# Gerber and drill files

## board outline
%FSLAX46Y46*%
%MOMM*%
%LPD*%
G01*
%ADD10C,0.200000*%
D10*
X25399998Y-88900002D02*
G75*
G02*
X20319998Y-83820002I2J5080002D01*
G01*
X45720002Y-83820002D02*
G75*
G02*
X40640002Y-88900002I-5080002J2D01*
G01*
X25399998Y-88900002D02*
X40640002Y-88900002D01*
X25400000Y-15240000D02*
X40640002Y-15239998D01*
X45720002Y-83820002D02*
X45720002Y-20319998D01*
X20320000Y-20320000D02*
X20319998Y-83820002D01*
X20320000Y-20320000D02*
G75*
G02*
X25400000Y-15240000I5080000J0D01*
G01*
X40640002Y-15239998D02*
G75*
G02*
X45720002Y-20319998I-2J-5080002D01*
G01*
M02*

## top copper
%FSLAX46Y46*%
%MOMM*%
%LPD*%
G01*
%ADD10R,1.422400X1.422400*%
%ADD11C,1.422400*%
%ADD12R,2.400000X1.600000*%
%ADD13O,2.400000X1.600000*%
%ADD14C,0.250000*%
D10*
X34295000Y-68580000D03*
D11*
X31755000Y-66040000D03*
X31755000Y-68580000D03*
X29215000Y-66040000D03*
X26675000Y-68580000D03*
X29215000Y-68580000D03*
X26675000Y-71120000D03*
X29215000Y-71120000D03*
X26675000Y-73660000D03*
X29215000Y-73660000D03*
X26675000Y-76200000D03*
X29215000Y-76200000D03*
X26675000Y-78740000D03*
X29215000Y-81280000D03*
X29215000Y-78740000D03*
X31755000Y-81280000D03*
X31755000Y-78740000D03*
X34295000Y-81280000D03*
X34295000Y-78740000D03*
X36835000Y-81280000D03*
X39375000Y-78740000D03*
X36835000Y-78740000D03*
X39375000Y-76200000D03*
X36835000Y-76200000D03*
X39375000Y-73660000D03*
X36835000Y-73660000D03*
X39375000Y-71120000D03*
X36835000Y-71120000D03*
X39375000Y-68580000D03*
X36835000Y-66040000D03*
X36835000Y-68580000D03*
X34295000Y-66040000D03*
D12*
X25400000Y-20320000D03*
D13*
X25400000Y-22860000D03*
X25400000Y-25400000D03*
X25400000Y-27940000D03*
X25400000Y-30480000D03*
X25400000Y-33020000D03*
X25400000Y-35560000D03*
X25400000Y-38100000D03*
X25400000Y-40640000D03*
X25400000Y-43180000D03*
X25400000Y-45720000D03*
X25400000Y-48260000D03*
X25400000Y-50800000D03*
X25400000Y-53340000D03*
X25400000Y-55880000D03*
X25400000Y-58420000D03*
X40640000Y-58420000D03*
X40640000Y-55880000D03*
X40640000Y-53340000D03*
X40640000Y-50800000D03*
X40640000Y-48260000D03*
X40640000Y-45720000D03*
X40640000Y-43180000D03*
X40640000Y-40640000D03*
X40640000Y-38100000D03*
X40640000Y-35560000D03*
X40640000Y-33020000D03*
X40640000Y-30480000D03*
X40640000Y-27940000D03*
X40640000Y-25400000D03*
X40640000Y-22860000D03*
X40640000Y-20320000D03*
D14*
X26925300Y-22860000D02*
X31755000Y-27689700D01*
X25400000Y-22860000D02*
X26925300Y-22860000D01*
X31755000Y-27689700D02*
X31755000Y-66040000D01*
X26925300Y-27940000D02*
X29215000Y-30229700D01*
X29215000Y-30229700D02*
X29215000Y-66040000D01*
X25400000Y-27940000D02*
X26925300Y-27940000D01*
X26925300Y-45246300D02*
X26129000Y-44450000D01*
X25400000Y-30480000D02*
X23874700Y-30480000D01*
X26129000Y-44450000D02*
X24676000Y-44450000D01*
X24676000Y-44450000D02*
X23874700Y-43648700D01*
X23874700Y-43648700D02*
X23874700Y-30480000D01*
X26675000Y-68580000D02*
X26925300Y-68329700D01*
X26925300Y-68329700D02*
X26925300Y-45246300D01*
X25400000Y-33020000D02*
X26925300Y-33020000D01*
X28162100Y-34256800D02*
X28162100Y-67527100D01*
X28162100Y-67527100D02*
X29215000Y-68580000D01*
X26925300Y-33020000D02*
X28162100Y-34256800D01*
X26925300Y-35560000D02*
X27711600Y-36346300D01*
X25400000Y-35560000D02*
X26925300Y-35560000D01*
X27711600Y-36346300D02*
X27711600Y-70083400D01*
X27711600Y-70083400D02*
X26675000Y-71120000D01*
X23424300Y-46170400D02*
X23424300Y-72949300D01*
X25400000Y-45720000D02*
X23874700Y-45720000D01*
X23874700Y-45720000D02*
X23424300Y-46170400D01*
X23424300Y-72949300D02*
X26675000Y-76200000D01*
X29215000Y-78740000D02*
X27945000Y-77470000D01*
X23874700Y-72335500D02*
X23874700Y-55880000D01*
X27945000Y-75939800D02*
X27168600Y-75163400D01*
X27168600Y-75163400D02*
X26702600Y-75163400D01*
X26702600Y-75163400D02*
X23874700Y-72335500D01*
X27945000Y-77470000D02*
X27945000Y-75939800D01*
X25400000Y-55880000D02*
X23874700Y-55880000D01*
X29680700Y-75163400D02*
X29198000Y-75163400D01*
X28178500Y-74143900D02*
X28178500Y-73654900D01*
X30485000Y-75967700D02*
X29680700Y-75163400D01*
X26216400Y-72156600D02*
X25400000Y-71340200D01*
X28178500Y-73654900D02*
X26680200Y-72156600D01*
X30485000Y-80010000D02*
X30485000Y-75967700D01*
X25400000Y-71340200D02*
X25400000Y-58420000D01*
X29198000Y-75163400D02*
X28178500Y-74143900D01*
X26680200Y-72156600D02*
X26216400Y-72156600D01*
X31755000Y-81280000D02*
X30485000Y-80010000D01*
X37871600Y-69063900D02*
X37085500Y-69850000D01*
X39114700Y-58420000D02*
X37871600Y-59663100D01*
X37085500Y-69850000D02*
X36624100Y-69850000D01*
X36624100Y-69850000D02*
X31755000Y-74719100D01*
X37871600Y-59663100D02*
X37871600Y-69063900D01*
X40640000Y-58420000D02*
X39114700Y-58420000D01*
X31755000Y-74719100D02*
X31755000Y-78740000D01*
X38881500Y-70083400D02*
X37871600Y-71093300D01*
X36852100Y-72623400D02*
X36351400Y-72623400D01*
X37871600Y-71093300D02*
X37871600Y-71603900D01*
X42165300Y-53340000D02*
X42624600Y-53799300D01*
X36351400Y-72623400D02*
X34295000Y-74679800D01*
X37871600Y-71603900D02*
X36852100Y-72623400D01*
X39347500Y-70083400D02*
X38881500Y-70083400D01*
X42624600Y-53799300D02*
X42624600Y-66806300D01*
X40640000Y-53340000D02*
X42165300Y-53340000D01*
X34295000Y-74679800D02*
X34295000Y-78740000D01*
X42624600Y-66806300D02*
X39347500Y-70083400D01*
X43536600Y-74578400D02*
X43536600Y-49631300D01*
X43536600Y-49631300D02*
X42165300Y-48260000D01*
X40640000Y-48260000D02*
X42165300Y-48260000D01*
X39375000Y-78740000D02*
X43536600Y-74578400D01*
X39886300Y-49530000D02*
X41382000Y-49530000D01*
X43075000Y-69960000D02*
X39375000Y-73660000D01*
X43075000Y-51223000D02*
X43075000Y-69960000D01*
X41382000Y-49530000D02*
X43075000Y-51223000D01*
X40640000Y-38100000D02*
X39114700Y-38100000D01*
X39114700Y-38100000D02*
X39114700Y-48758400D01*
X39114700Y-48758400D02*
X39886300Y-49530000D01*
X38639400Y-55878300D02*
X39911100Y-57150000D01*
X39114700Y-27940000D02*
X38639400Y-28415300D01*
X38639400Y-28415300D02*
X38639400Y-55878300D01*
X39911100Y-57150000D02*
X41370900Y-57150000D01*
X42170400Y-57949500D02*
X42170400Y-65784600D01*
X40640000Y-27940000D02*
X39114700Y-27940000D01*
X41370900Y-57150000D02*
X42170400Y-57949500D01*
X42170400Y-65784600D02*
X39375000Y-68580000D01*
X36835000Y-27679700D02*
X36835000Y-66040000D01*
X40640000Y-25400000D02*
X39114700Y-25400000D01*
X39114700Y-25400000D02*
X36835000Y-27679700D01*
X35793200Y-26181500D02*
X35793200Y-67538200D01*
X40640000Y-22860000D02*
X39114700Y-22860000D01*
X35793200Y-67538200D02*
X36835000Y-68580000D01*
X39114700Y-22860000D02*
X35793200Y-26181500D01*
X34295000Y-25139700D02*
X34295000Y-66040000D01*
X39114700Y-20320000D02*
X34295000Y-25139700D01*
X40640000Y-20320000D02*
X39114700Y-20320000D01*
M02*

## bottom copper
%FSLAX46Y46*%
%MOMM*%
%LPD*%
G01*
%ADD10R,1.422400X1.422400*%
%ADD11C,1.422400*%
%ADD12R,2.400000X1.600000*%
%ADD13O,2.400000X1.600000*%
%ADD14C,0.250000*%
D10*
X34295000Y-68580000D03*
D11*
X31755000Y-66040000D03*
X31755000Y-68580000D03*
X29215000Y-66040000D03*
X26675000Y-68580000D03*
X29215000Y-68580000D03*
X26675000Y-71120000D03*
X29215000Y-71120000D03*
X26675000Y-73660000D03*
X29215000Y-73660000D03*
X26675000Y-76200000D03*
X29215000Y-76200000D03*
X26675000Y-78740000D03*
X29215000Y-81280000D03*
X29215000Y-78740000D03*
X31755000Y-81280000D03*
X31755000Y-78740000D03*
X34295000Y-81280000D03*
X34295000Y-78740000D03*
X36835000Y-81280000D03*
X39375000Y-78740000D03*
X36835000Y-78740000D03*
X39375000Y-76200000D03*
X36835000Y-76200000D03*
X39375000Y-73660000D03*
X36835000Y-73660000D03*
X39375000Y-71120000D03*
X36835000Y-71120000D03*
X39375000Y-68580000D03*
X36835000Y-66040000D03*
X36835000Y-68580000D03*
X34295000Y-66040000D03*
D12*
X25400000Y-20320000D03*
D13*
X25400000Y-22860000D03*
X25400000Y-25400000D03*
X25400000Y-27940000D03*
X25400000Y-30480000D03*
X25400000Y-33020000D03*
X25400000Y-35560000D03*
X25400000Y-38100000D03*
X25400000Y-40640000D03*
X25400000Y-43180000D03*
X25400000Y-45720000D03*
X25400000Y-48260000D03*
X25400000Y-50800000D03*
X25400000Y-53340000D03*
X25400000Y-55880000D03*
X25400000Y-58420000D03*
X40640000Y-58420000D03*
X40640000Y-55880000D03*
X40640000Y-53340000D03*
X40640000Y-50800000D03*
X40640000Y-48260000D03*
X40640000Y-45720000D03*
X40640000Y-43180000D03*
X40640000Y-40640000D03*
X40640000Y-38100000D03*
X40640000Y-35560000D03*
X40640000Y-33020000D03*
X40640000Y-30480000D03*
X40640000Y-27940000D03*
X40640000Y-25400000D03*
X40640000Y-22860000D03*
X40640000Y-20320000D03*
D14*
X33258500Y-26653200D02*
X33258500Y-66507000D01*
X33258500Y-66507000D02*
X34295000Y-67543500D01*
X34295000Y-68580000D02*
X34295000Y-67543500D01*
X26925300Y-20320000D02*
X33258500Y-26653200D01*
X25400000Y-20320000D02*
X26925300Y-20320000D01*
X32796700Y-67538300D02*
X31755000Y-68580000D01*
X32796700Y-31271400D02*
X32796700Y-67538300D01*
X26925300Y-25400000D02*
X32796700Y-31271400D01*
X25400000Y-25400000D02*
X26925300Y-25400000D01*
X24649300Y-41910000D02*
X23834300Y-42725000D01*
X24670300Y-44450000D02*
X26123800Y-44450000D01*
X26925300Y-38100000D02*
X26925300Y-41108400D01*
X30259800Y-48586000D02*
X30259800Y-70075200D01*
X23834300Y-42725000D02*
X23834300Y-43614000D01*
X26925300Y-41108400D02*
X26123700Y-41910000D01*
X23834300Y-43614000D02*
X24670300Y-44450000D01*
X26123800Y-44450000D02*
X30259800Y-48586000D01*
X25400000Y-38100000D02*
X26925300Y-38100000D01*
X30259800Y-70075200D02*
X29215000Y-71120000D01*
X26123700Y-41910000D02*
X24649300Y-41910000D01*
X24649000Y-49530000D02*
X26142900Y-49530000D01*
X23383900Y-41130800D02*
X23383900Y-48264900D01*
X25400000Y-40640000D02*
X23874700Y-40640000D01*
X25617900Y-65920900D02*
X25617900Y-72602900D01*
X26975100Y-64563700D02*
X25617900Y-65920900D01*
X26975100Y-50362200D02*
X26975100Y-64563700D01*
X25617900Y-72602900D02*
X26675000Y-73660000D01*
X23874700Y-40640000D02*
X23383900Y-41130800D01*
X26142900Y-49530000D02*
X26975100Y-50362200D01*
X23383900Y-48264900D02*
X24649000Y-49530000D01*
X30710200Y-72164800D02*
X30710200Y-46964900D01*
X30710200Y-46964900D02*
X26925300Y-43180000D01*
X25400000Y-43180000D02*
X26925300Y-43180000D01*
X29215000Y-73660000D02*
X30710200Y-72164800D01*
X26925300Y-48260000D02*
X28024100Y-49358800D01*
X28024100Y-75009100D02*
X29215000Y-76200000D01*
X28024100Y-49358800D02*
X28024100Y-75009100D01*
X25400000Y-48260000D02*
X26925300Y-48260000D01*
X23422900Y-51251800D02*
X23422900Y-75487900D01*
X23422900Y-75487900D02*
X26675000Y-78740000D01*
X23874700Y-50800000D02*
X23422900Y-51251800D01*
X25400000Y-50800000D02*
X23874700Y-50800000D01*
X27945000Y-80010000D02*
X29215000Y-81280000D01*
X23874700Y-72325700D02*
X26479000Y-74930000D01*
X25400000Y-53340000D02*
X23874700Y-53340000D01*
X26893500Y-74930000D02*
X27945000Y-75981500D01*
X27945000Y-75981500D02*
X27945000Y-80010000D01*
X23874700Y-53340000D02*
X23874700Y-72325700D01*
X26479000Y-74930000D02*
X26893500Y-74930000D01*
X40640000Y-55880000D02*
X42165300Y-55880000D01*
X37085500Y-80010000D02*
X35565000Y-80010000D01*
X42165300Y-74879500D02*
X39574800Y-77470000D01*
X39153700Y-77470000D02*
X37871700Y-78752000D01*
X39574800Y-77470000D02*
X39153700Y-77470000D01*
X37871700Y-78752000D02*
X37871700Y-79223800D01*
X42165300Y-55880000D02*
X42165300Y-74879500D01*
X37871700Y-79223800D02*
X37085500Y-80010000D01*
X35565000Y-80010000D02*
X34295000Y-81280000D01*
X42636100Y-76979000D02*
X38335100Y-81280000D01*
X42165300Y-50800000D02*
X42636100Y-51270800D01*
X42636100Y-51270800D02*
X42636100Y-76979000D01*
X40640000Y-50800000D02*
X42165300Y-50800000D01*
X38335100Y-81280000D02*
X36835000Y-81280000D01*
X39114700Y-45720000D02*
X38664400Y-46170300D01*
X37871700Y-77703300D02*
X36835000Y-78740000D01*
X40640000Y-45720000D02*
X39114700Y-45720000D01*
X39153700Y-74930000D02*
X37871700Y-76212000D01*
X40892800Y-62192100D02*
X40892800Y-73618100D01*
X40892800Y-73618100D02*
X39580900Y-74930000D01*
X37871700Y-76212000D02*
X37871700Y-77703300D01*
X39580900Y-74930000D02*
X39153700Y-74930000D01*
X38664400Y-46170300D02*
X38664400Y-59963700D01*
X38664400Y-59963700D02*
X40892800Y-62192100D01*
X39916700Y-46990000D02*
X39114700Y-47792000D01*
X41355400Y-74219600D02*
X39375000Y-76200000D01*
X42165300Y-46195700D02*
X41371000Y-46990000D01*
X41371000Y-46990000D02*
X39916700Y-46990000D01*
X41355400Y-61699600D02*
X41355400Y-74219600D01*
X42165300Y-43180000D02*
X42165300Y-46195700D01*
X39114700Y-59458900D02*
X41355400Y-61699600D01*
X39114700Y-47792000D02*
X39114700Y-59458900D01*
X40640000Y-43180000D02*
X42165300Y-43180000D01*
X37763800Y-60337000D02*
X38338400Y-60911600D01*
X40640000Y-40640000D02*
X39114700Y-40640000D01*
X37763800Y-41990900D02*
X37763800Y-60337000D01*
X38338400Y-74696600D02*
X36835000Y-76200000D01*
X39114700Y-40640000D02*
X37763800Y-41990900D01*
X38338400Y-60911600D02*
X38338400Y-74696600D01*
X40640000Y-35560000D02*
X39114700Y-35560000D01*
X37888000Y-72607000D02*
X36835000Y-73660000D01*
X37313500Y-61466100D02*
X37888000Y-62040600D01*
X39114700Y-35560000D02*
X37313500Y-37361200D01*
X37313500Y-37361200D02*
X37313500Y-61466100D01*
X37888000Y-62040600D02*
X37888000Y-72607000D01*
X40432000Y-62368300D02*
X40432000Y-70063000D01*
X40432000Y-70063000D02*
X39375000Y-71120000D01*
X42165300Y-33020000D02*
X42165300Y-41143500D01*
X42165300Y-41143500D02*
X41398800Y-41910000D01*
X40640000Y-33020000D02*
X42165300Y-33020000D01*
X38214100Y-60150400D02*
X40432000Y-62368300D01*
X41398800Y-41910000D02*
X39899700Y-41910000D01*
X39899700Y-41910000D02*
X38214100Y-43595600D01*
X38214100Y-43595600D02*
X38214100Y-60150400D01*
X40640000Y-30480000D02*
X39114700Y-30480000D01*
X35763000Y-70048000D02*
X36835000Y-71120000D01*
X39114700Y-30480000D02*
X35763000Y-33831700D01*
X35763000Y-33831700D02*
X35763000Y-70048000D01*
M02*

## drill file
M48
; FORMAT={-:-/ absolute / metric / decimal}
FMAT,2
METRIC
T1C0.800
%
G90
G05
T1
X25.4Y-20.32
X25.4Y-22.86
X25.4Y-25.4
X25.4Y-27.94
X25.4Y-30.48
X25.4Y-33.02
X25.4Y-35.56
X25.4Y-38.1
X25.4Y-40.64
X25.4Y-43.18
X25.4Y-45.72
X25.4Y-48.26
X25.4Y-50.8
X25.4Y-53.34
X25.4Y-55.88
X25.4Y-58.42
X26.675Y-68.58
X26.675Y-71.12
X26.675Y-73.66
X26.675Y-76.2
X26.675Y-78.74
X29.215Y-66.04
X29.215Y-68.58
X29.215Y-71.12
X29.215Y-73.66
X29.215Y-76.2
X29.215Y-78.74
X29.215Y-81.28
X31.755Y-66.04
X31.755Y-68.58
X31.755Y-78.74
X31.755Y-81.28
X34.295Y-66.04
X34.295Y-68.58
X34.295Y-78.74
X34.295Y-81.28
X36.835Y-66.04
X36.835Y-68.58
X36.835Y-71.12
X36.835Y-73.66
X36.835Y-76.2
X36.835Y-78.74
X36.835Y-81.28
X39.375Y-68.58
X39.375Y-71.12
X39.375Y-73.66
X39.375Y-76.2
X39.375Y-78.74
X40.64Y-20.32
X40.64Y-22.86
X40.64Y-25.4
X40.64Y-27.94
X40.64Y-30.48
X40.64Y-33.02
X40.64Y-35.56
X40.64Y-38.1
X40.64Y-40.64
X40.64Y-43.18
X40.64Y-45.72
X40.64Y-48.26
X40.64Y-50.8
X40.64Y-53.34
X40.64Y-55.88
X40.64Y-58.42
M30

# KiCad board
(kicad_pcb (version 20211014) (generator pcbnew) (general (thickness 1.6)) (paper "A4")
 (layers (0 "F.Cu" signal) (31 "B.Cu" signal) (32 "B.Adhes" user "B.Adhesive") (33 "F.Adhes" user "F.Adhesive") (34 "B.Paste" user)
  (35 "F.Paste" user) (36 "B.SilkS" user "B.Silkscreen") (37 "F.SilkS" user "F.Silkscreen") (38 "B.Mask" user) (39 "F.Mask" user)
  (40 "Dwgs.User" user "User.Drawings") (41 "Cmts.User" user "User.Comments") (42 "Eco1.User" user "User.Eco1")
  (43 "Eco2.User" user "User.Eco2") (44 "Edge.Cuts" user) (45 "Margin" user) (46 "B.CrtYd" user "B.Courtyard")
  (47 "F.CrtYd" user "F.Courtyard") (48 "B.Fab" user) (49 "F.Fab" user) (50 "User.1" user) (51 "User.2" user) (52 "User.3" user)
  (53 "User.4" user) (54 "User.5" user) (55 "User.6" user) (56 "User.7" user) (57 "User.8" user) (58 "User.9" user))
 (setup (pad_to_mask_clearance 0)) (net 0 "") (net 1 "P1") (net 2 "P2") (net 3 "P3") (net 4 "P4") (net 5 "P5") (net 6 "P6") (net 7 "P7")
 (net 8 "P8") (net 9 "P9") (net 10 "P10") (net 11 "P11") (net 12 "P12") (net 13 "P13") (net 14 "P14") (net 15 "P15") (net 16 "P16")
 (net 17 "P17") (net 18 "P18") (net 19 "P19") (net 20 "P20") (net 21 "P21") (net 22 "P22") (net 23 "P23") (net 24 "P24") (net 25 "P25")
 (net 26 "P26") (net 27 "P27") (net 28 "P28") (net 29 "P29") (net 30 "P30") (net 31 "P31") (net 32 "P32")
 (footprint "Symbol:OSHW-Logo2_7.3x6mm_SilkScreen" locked (layer "F.Cu") (at 31.496 49.784 -90)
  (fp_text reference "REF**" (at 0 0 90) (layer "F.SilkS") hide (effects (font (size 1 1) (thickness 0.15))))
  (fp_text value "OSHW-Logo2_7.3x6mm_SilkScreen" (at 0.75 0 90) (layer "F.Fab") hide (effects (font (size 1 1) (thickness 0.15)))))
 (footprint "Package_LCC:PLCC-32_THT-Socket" (layer "F.Cu") (at 34.295 68.58)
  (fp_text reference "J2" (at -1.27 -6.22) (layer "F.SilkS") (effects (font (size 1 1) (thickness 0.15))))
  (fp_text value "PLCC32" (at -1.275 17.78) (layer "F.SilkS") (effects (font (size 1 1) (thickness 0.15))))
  (pad "1" thru_hole rect (at 0 0) (size 1.4224 1.4224) (drill 0.8) (layers *.Cu *.Mask) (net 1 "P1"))
  (pad "2" thru_hole circle (at -2.54 -2.54) (size 1.4224 1.4224) (drill 0.8) (layers *.Cu *.Mask) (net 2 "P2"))
  (pad "3" thru_hole circle (at -2.54 0) (size 1.4224 1.4224) (drill 0.8) (layers *.Cu *.Mask) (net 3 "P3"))
  (pad "4" thru_hole circle (at -5.08 -2.54) (size 1.4224 1.4224) (drill 0.8) (layers *.Cu *.Mask) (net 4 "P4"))
  (pad "5" thru_hole circle (at -7.62 0) (size 1.4224 1.4224) (drill 0.8) (layers *.Cu *.Mask) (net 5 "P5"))
  (pad "6" thru_hole circle (at -5.08 0) (size 1.4224 1.4224) (drill 0.8) (layers *.Cu *.Mask) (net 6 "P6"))
  (pad "7" thru_hole circle (at -7.62 2.54) (size 1.4224 1.4224) (drill 0.8) (layers *.Cu *.Mask) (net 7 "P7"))
  (pad "8" thru_hole circle (at -5.08 2.54) (size 1.4224 1.4224) (drill 0.8) (layers *.Cu *.Mask) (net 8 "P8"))
  (pad "9" thru_hole circle (at -7.62 5.08) (size 1.4224 1.4224) (drill 0.8) (layers *.Cu *.Mask) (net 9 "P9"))
  (pad "10" thru_hole circle (at -5.08 5.08) (size 1.4224 1.4224) (drill 0.8) (layers *.Cu *.Mask) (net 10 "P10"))
  (pad "11" thru_hole circle (at -7.62 7.62) (size 1.4224 1.4224) (drill 0.8) (layers *.Cu *.Mask) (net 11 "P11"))
  (pad "12" thru_hole circle (at -5.08 7.62) (size 1.4224 1.4224) (drill 0.8) (layers *.Cu *.Mask) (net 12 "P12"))
  (pad "13" thru_hole circle (at -7.62 10.16) (size 1.4224 1.4224) (drill 0.8) (layers *.Cu *.Mask) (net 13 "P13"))
  (pad "14" thru_hole circle (at -5.08 12.7) (size 1.4224 1.4224) (drill 0.8) (layers *.Cu *.Mask) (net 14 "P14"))
  (pad "15" thru_hole circle (at -5.08 10.16) (size 1.4224 1.4224) (drill 0.8) (layers *.Cu *.Mask) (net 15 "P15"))
  (pad "16" thru_hole circle (at -2.54 12.7) (size 1.4224 1.4224) (drill 0.8) (layers *.Cu *.Mask) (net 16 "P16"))
  (pad "17" thru_hole circle (at -2.54 10.16) (size 1.4224 1.4224) (drill 0.8) (layers *.Cu *.Mask) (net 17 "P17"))
  (pad "18" thru_hole circle (at 0 12.7) (size 1.4224 1.4224) (drill 0.8) (layers *.Cu *.Mask) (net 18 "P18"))
  (pad "19" thru_hole circle (at 0 10.16) (size 1.4224 1.4224) (drill 0.8) (layers *.Cu *.Mask) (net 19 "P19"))
  (pad "20" thru_hole circle (at 2.54 12.7) (size 1.4224 1.4224) (drill 0.8) (layers *.Cu *.Mask) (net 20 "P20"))
  (pad "21" thru_hole circle (at 5.08 10.16) (size 1.4224 1.4224) (drill 0.8) (layers *.Cu *.Mask) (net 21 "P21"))
  (pad "22" thru_hole circle (at 2.54 10.16) (size 1.4224 1.4224) (drill 0.8) (layers *.Cu *.Mask) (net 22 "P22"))
  (pad "23" thru_hole circle (at 5.08 7.62) (size 1.4224 1.4224) (drill 0.8) (layers *.Cu *.Mask) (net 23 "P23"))
  (pad "24" thru_hole circle (at 2.54 7.62) (size 1.4224 1.4224) (drill 0.8) (layers *.Cu *.Mask) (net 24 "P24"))
  (pad "25" thru_hole circle (at 5.08 5.08) (size 1.4224 1.4224) (drill 0.8) (layers *.Cu *.Mask) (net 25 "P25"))
  (pad "26" thru_hole circle (at 2.54 5.08) (size 1.4224 1.4224) (drill 0.8) (layers *.Cu *.Mask) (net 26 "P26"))
  (pad "27" thru_hole circle (at 5.08 2.54) (size 1.4224 1.4224) (drill 0.8) (layers *.Cu *.Mask) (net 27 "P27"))
  (pad "28" thru_hole circle (at 2.54 2.54) (size 1.4224 1.4224) (drill 0.8) (layers *.Cu *.Mask) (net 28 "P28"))
  (pad "29" thru_hole circle (at 5.08 0) (size 1.4224 1.4224) (drill 0.8) (layers *.Cu *.Mask) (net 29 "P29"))
  (pad "30" thru_hole circle (at 2.54 -2.54) (size 1.4224 1.4224) (drill 0.8) (layers *.Cu *.Mask) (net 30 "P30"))
  (pad "31" thru_hole circle (at 2.54 0) (size 1.4224 1.4224) (drill 0.8) (layers *.Cu *.Mask) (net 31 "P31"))
  (pad "32" thru_hole circle (at 0 -2.54) (size 1.4224 1.4224) (drill 0.8) (layers *.Cu *.Mask) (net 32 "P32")))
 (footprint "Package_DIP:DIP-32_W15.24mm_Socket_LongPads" (layer "F.Cu") (at 25.4 20.32)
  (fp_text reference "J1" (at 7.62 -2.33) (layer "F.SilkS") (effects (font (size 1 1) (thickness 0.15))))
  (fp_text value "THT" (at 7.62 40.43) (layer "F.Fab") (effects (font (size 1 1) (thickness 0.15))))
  (pad "1" thru_hole rect (at 0 0) (size 2.4 1.6) (drill 0.8) (layers *.Cu *.Mask) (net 1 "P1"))
  (pad "2" thru_hole oval (at 0 2.54) (size 2.4 1.6) (drill 0.8) (layers *.Cu *.Mask) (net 2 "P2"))
  (pad "3" thru_hole oval (at 0 5.08) (size 2.4 1.6) (drill 0.8) (layers *.Cu *.Mask) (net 3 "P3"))
  (pad "4" thru_hole oval (at 0 7.62) (size 2.4 1.6) (drill 0.8) (layers *.Cu *.Mask) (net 4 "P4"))
  (pad "5" thru_hole oval (at 0 10.16) (size 2.4 1.6) (drill 0.8) (layers *.Cu *.Mask) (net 5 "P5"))
  (pad "6" thru_hole oval (at 0 12.7) (size 2.4 1.6) (drill 0.8) (layers *.Cu *.Mask) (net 6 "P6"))
  (pad "7" thru_hole oval (at 0 15.24) (size 2.4 1.6) (drill 0.8) (layers *.Cu *.Mask) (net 7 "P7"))
  (pad "8" thru_hole oval (at 0 17.78) (size 2.4 1.6) (drill 0.8) (layers *.Cu *.Mask) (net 8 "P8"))
  (pad "9" thru_hole oval (at 0 20.32) (size 2.4 1.6) (drill 0.8) (layers *.Cu *.Mask) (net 9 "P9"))
  (pad "10" thru_hole oval (at 0 22.86) (size 2.4 1.6) (drill 0.8) (layers *.Cu *.Mask) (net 10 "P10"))
  (pad "11" thru_hole oval (at 0 25.4) (size 2.4 1.6) (drill 0.8) (layers *.Cu *.Mask) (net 11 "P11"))
  (pad "12" thru_hole oval (at 0 27.94) (size 2.4 1.6) (drill 0.8) (layers *.Cu *.Mask) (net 12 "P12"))
  (pad "13" thru_hole oval (at 0 30.48) (size 2.4 1.6) (drill 0.8) (layers *.Cu *.Mask) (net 13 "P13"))
  (pad "14" thru_hole oval (at 0 33.02) (size 2.4 1.6) (drill 0.8) (layers *.Cu *.Mask) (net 14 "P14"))
  (pad "15" thru_hole oval (at 0 35.56) (size 2.4 1.6) (drill 0.8) (layers *.Cu *.Mask) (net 15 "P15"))
  (pad "16" thru_hole oval (at 0 38.1) (size 2.4 1.6) (drill 0.8) (layers *.Cu *.Mask) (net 16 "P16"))
  (pad "17" thru_hole oval (at 15.24 38.1) (size 2.4 1.6) (drill 0.8) (layers *.Cu *.Mask) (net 17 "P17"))
  (pad "18" thru_hole oval (at 15.24 35.56) (size 2.4 1.6) (drill 0.8) (layers *.Cu *.Mask) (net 18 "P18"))
  (pad "19" thru_hole oval (at 15.24 33.02) (size 2.4 1.6) (drill 0.8) (layers *.Cu *.Mask) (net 19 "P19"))
  (pad "20" thru_hole oval (at 15.24 30.48) (size 2.4 1.6) (drill 0.8) (layers *.Cu *.Mask) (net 20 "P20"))
  (pad "21" thru_hole oval (at 15.24 27.94) (size 2.4 1.6) (drill 0.8) (layers *.Cu *.Mask) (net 21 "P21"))
  (pad "22" thru_hole oval (at 15.24 25.4) (size 2.4 1.6) (drill 0.8) (layers *.Cu *.Mask) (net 22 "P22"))
  (pad "23" thru_hole oval (at 15.24 22.86) (size 2.4 1.6) (drill 0.8) (layers *.Cu *.Mask) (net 23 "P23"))
  (pad "24" thru_hole oval (at 15.24 20.32) (size 2.4 1.6) (drill 0.8) (layers *.Cu *.Mask) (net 24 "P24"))
  (pad "25" thru_hole oval (at 15.24 17.78) (size 2.4 1.6) (drill 0.8) (layers *.Cu *.Mask) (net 25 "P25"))
  (pad "26" thru_hole oval (at 15.24 15.24) (size 2.4 1.6) (drill 0.8) (layers *.Cu *.Mask) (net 26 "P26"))
  (pad "27" thru_hole oval (at 15.24 12.7) (size 2.4 1.6) (drill 0.8) (layers *.Cu *.Mask) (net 27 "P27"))
  (pad "28" thru_hole oval (at 15.24 10.16) (size 2.4 1.6) (drill 0.8) (layers *.Cu *.Mask) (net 28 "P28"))
  (pad "29" thru_hole oval (at 15.24 7.62) (size 2.4 1.6) (drill 0.8) (layers *.Cu *.Mask) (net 29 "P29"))
  (pad "30" thru_hole oval (at 15.24 5.08) (size 2.4 1.6) (drill 0.8) (layers *.Cu *.Mask) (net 30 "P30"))
  (pad "31" thru_hole oval (at 15.24 2.54) (size 2.4 1.6) (drill 0.8) (layers *.Cu *.Mask) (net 31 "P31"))
  (pad "32" thru_hole oval (at 15.24 0) (size 2.4 1.6) (drill 0.8) (layers *.Cu *.Mask) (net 32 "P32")))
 (gr_arc (start 25.399998 88.900002) (mid 21.807896 87.412104) (end 20.319998 83.820002) (layer "Edge.Cuts") (width 0.2))
 (gr_arc (start 45.720002 83.820002) (mid 44.232104 87.412104) (end 40.640002 88.900002) (layer "Edge.Cuts") (width 0.2))
 (gr_line (start 25.399998 88.900002) (end 40.640002 88.900002) (layer "Edge.Cuts") (width 0.2))
 (gr_line (start 25.4 15.24) (end 40.640002 15.239998) (layer "Edge.Cuts") (width 0.2))
 (gr_line (start 45.720002 83.820002) (end 45.720002 20.319998) (layer "Edge.Cuts") (width 0.2))
 (gr_line (start 20.32 20.32) (end 20.319998 83.820002) (layer "Edge.Cuts") (width 0.2))
 (gr_arc (start 20.32 20.32) (mid 21.807898 16.727898) (end 25.4 15.24) (layer "Edge.Cuts") (width 0.2))
 (gr_arc (start 40.640002 15.239998) (mid 44.232104 16.727896) (end 45.720002 20.319998) (layer "Edge.Cuts") (width 0.2))
 (segment (start 33.2585 26.6532) (end 33.2585 66.507) (width 0.25) (layer "B.Cu") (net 1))
 (segment (start 33.2585 66.507) (end 34.295 67.5435) (width 0.25) (layer "B.Cu") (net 1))
 (segment (start 34.295 68.58) (end 34.295 67.5435) (width 0.25) (layer "B.Cu") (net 1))
 (segment (start 26.9253 20.32) (end 33.2585 26.6532) (width 0.25) (layer "B.Cu") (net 1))
 (segment (start 25.4 20.32) (end 26.9253 20.32) (width 0.25) (layer "B.Cu") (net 1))
 (segment (start 26.9253 22.86) (end 31.755 27.6897) (width 0.25) (layer "F.Cu") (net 2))
 (segment (start 25.4 22.86) (end 26.9253 22.86) (width 0.25) (layer "F.Cu") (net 2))
 (segment (start 31.755 27.6897) (end 31.755 66.04) (width 0.25) (layer "F.Cu") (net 2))
 (segment (start 32.7967 67.5383) (end 31.755 68.58) (width 0.25) (layer "B.Cu") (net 3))
 (segment (start 32.7967 31.2714) (end 32.7967 67.5383) (width 0.25) (layer "B.Cu") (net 3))
 (segment (start 26.9253 25.4) (end 32.7967 31.2714) (width 0.25) (layer "B.Cu") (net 3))
 (segment (start 25.4 25.4) (end 26.9253 25.4) (width 0.25) (layer "B.Cu") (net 3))
 (segment (start 26.9253 27.94) (end 29.215 30.2297) (width 0.25) (layer "F.Cu") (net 4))
 (segment (start 29.215 30.2297) (end 29.215 66.04) (width 0.25) (layer "F.Cu") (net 4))
 (segment (start 25.4 27.94) (end 26.9253 27.94) (width 0.25) (layer "F.Cu") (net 4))
 (segment (start 26.9253 45.2463) (end 26.129 44.45) (width 0.25) (layer "F.Cu") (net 5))
 (segment (start 25.4 30.48) (end 23.8747 30.48) (width 0.25) (layer "F.Cu") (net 5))
 (segment (start 26.129 44.45) (end 24.676 44.45) (width 0.25) (layer "F.Cu") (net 5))
 (segment (start 24.676 44.45) (end 23.8747 43.6487) (width 0.25) (layer "F.Cu") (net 5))
 (segment (start 23.8747 43.6487) (end 23.8747 30.48) (width 0.25) (layer "F.Cu") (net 5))
 (segment (start 26.675 68.58) (end 26.9253 68.3297) (width 0.25) (layer "F.Cu") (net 5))
 (segment (start 26.9253 68.3297) (end 26.9253 45.2463) (width 0.25) (layer "F.Cu") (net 5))
 (segment (start 25.4 33.02) (end 26.9253 33.02) (width 0.25) (layer "F.Cu") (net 6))
 (segment (start 28.1621 34.2568) (end 28.1621 67.5271) (width 0.25) (layer "F.Cu") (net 6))
 (segment (start 28.1621 67.5271) (end 29.215 68.58) (width 0.25) (layer "F.Cu") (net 6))
 (segment (start 26.9253 33.02) (end 28.1621 34.2568) (width 0.25) (layer "F.Cu") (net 6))
 (segment (start 26.9253 35.56) (end 27.7116 36.3463) (width 0.25) (layer "F.Cu") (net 7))
 (segment (start 25.4 35.56) (end 26.9253 35.56) (width 0.25) (layer "F.Cu") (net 7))
 (segment (start 27.7116 36.3463) (end 27.7116 70.0834) (width 0.25) (layer "F.Cu") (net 7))
 (segment (start 27.7116 70.0834) (end 26.675 71.12) (width 0.25) (layer "F.Cu") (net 7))
 (segment (start 24.6493 41.91) (end 23.8343 42.725) (width 0.25) (layer "B.Cu") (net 8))
 (segment (start 24.6703 44.45) (end 26.1238 44.45) (width 0.25) (layer "B.Cu") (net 8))
 (segment (start 26.9253 38.1) (end 26.9253 41.1084) (width 0.25) (layer "B.Cu") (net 8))
 (segment (start 30.2598 48.586) (end 30.2598 70.0752) (width 0.25) (layer "B.Cu") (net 8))
 (segment (start 23.8343 42.725) (end 23.8343 43.614) (width 0.25) (layer "B.Cu") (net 8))
 (segment (start 26.9253 41.1084) (end 26.1237 41.91) (width 0.25) (layer "B.Cu") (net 8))
 (segment (start 23.8343 43.614) (end 24.6703 44.45) (width 0.25) (layer "B.Cu") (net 8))
 (segment (start 26.1238 44.45) (end 30.2598 48.586) (width 0.25) (layer "B.Cu") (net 8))
 (segment (start 25.4 38.1) (end 26.9253 38.1) (width 0.25) (layer "B.Cu") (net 8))
 (segment (start 30.2598 70.0752) (end 29.215 71.12) (width 0.25) (layer "B.Cu") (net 8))
 (segment (start 26.1237 41.91) (end 24.6493 41.91) (width 0.25) (layer "B.Cu") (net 8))
 (segment (start 24.649 49.53) (end 26.1429 49.53) (width 0.25) (layer "B.Cu") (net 9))
 (segment (start 23.3839 41.1308) (end 23.3839 48.2649) (width 0.25) (layer "B.Cu") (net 9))
 (segment (start 25.4 40.64) (end 23.8747 40.64) (width 0.25) (layer "B.Cu") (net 9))
 (segment (start 25.6179 65.9209) (end 25.6179 72.6029) (width 0.25) (layer "B.Cu") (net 9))
 (segment (start 26.9751 64.5637) (end 25.6179 65.9209) (width 0.25) (layer "B.Cu") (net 9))
 (segment (start 26.9751 50.3622) (end 26.9751 64.5637) (width 0.25) (layer "B.Cu") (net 9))
 (segment (start 25.6179 72.6029) (end 26.675 73.66) (width 0.25) (layer "B.Cu") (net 9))
 (segment (start 23.8747 40.64) (end 23.3839 41.1308) (width 0.25) (layer "B.Cu") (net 9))
 (segment (start 26.1429 49.53) (end 26.9751 50.3622) (width 0.25) (layer "B.Cu") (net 9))
 (segment (start 23.3839 48.2649) (end 24.649 49.53) (width 0.25) (layer "B.Cu") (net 9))
 (segment (start 30.7102 72.1648) (end 30.7102 46.9649) (width 0.25) (layer "B.Cu") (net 10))
 (segment (start 30.7102 46.9649) (end 26.9253 43.18) (width 0.25) (layer "B.Cu") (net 10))
 (segment (start 25.4 43.18) (end 26.9253 43.18) (width 0.25) (layer "B.Cu") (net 10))
 (segment (start 29.215 73.66) (end 30.7102 72.1648) (width 0.25) (layer "B.Cu") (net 10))
 (segment (start 23.4243 46.1704) (end 23.4243 72.9493) (width 0.25) (layer "F.Cu") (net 11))
 (segment (start 25.4 45.72) (end 23.8747 45.72) (width 0.25) (layer "F.Cu") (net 11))
 (segment (start 23.8747 45.72) (end 23.4243 46.1704) (width 0.25) (layer "F.Cu") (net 11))
 (segment (start 23.4243 72.9493) (end 26.675 76.2) (width 0.25) (layer "F.Cu") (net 11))
 (segment (start 26.9253 48.26) (end 28.0241 49.3588) (width 0.25) (layer "B.Cu") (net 12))
 (segment (start 28.0241 75.0091) (end 29.215 76.2) (width 0.25) (layer "B.Cu") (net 12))
 (segment (start 28.0241 49.3588) (end 28.0241 75.0091) (width 0.25) (layer "B.Cu") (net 12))
 (segment (start 25.4 48.26) (end 26.9253 48.26) (width 0.25) (layer "B.Cu") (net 12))
 (segment (start 23.4229 51.2518) (end 23.4229 75.4879) (width 0.25) (layer "B.Cu") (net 13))
 (segment (start 23.4229 75.4879) (end 26.675 78.74) (width 0.25) (layer "B.Cu") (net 13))
 (segment (start 23.8747 50.8) (end 23.4229 51.2518) (width 0.25) (layer "B.Cu") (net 13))
 (segment (start 25.4 50.8) (end 23.8747 50.8) (width 0.25) (layer "B.Cu") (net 13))
 (segment (start 27.945 80.01) (end 29.215 81.28) (width 0.25) (layer "B.Cu") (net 14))
 (segment (start 23.8747 72.3257) (end 26.479 74.93) (width 0.25) (layer "B.Cu") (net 14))
 (segment (start 25.4 53.34) (end 23.8747 53.34) (width 0.25) (layer "B.Cu") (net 14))
 (segment (start 26.8935 74.93) (end 27.945 75.9815) (width 0.25) (layer "B.Cu") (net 14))
 (segment (start 27.945 75.9815) (end 27.945 80.01) (width 0.25) (layer "B.Cu") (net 14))
 (segment (start 23.8747 53.34) (end 23.8747 72.3257) (width 0.25) (layer "B.Cu") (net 14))
 (segment (start 26.479 74.93) (end 26.8935 74.93) (width 0.25) (layer "B.Cu") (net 14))
 (segment (start 29.215 78.74) (end 27.945 77.47) (width 0.25) (layer "F.Cu") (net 15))
 (segment (start 23.8747 72.3355) (end 23.8747 55.88) (width 0.25) (layer "F.Cu") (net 15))
 (segment (start 27.945 75.9398) (end 27.1686 75.1634) (width 0.25) (layer "F.Cu") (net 15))
 (segment (start 27.1686 75.1634) (end 26.7026 75.1634) (width 0.25) (layer "F.Cu") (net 15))
 (segment (start 26.7026 75.1634) (end 23.8747 72.3355) (width 0.25) (layer "F.Cu") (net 15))
 (segment (start 27.945 77.47) (end 27.945 75.9398) (width 0.25) (layer "F.Cu") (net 15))
 (segment (start 25.4 55.88) (end 23.8747 55.88) (width 0.25) (layer "F.Cu") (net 15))
 (segment (start 29.6807 75.1634) (end 29.198 75.1634) (width 0.25) (layer "F.Cu") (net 16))
 (segment (start 28.1785 74.1439) (end 28.1785 73.6549) (width 0.25) (layer "F.Cu") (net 16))
 (segment (start 30.485 75.9677) (end 29.6807 75.1634) (width 0.25) (layer "F.Cu") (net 16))
 (segment (start 26.2164 72.1566) (end 25.4 71.3402) (width 0.25) (layer "F.Cu") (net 16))
 (segment (start 28.1785 73.6549) (end 26.6802 72.1566) (width 0.25) (layer "F.Cu") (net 16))
 (segment (start 30.485 80.01) (end 30.485 75.9677) (width 0.25) (layer "F.Cu") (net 16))
 (segment (start 25.4 71.3402) (end 25.4 58.42) (width 0.25) (layer "F.Cu") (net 16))
 (segment (start 29.198 75.1634) (end 28.1785 74.1439) (width 0.25) (layer "F.Cu") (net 16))
 (segment (start 26.6802 72.1566) (end 26.2164 72.1566) (width 0.25) (layer "F.Cu") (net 16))
 (segment (start 31.755 81.28) (end 30.485 80.01) (width 0.25) (layer "F.Cu") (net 16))
 (segment (start 37.8716 69.0639) (end 37.0855 69.85) (width 0.25) (layer "F.Cu") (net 17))
 (segment (start 39.1147 58.42) (end 37.8716 59.6631) (width 0.25) (layer "F.Cu") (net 17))
 (segment (start 37.0855 69.85) (end 36.6241 69.85) (width 0.25) (layer "F.Cu") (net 17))
 (segment (start 36.6241 69.85) (end 31.755 74.7191) (width 0.25) (layer "F.Cu") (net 17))
 (segment (start 37.8716 59.6631) (end 37.8716 69.0639) (width 0.25) (layer "F.Cu") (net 17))
 (segment (start 40.64 58.42) (end 39.1147 58.42) (width 0.25) (layer "F.Cu") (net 17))
 (segment (start 31.755 74.7191) (end 31.755 78.74) (width 0.25) (layer "F.Cu") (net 17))
 (segment (start 40.64 55.88) (end 42.1653 55.88) (width 0.25) (layer "B.Cu") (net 18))
 (segment (start 37.0855 80.01) (end 35.565 80.01) (width 0.25) (layer "B.Cu") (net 18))
 (segment (start 42.1653 74.8795) (end 39.5748 77.47) (width 0.25) (layer "B.Cu") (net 18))
 (segment (start 39.1537 77.47) (end 37.8717 78.752) (width 0.25) (layer "B.Cu") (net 18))
 (segment (start 39.5748 77.47) (end 39.1537 77.47) (width 0.25) (layer "B.Cu") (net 18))
 (segment (start 37.8717 78.752) (end 37.8717 79.2238) (width 0.25) (layer "B.Cu") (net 18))
 (segment (start 42.1653 55.88) (end 42.1653 74.8795) (width 0.25) (layer "B.Cu") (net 18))
 (segment (start 37.8717 79.2238) (end 37.0855 80.01) (width 0.25) (layer "B.Cu") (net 18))
 (segment (start 35.565 80.01) (end 34.295 81.28) (width 0.25) (layer "B.Cu") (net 18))
 (segment (start 38.8815 70.0834) (end 37.8716 71.0933) (width 0.25) (layer "F.Cu") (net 19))
 (segment (start 36.8521 72.6234) (end 36.3514 72.6234) (width 0.25) (layer "F.Cu") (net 19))
 (segment (start 37.8716 71.0933) (end 37.8716 71.6039) (width 0.25) (layer "F.Cu") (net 19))
 (segment (start 42.1653 53.34) (end 42.6246 53.7993) (width 0.25) (layer "F.Cu") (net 19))
 (segment (start 36.3514 72.6234) (end 34.295 74.6798) (width 0.25) (layer "F.Cu") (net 19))
 (segment (start 37.8716 71.6039) (end 36.8521 72.6234) (width 0.25) (layer "F.Cu") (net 19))
 (segment (start 39.3475 70.0834) (end 38.8815 70.0834) (width 0.25) (layer "F.Cu") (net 19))
 (segment (start 42.6246 53.7993) (end 42.6246 66.8063) (width 0.25) (layer "F.Cu") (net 19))
 (segment (start 40.64 53.34) (end 42.1653 53.34) (width 0.25) (layer "F.Cu") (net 19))
 (segment (start 34.295 74.6798) (end 34.295 78.74) (width 0.25) (layer "F.Cu") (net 19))
 (segment (start 42.6246 66.8063) (end 39.3475 70.0834) (width 0.25) (layer "F.Cu") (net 19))
 (segment (start 42.6361 76.979) (end 38.3351 81.28) (width 0.25) (layer "B.Cu") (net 20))
 (segment (start 42.1653 50.8) (end 42.6361 51.2708) (width 0.25) (layer "B.Cu") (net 20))
 (segment (start 42.6361 51.2708) (end 42.6361 76.979) (width 0.25) (layer "B.Cu") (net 20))
 (segment (start 40.64 50.8) (end 42.1653 50.8) (width 0.25) (layer "B.Cu") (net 20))
 (segment (start 38.3351 81.28) (end 36.835 81.28) (width 0.25) (layer "B.Cu") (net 20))
 (segment (start 43.5366 74.5784) (end 43.5366 49.6313) (width 0.25) (layer "F.Cu") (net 21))
 (segment (start 43.5366 49.6313) (end 42.1653 48.26) (width 0.25) (layer "F.Cu") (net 21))
 (segment (start 40.64 48.26) (end 42.1653 48.26) (width 0.25) (layer "F.Cu") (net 21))
 (segment (start 39.375 78.74) (end 43.5366 74.5784) (width 0.25) (layer "F.Cu") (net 21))
 (segment (start 39.1147 45.72) (end 38.6644 46.1703) (width 0.25) (layer "B.Cu") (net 22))
 (segment (start 37.8717 77.7033) (end 36.835 78.74) (width 0.25) (layer "B.Cu") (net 22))
 (segment (start 40.64 45.72) (end 39.1147 45.72) (width 0.25) (layer "B.Cu") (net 22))
 (segment (start 39.1537 74.93) (end 37.8717 76.212) (width 0.25) (layer "B.Cu") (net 22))
 (segment (start 40.8928 62.1921) (end 40.8928 73.6181) (width 0.25) (layer "B.Cu") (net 22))
 (segment (start 40.8928 73.6181) (end 39.5809 74.93) (width 0.25) (layer "B.Cu") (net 22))
 (segment (start 37.8717 76.212) (end 37.8717 77.7033) (width 0.25) (layer "B.Cu") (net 22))
 (segment (start 39.5809 74.93) (end 39.1537 74.93) (width 0.25) (layer "B.Cu") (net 22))
 (segment (start 38.6644 46.1703) (end 38.6644 59.9637) (width 0.25) (layer "B.Cu") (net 22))
 (segment (start 38.6644 59.9637) (end 40.8928 62.1921) (width 0.25) (layer "B.Cu") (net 22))
 (segment (start 39.9167 46.99) (end 39.1147 47.792) (width 0.25) (layer "B.Cu") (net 23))
 (segment (start 41.3554 74.2196) (end 39.375 76.2) (width 0.25) (layer "B.Cu") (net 23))
 (segment (start 42.1653 46.1957) (end 41.371 46.99) (width 0.25) (layer "B.Cu") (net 23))
 (segment (start 41.371 46.99) (end 39.9167 46.99) (width 0.25) (layer "B.Cu") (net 23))
 (segment (start 41.3554 61.6996) (end 41.3554 74.2196) (width 0.25) (layer "B.Cu") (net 23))
 (segment (start 42.1653 43.18) (end 42.1653 46.1957) (width 0.25) (layer "B.Cu") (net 23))
 (segment (start 39.1147 59.4589) (end 41.3554 61.6996) (width 0.25) (layer "B.Cu") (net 23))
 (segment (start 39.1147 47.792) (end 39.1147 59.4589) (width 0.25) (layer "B.Cu") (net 23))
 (segment (start 40.64 43.18) (end 42.1653 43.18) (width 0.25) (layer "B.Cu") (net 23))
 (segment (start 37.7638 60.337) (end 38.3384 60.9116) (width 0.25) (layer "B.Cu") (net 24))
 (segment (start 40.64 40.64) (end 39.1147 40.64) (width 0.25) (layer "B.Cu") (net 24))
 (segment (start 37.7638 41.9909) (end 37.7638 60.337) (width 0.25) (layer "B.Cu") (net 24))
 (segment (start 38.3384 74.6966) (end 36.835 76.2) (width 0.25) (layer "B.Cu") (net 24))
 (segment (start 39.1147 40.64) (end 37.7638 41.9909) (width 0.25) (layer "B.Cu") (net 24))
 (segment (start 38.3384 60.9116) (end 38.3384 74.6966) (width 0.25) (layer "B.Cu") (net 24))
 (segment (start 39.8863 49.53) (end 41.382 49.53) (width 0.25) (layer "F.Cu") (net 25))
 (segment (start 43.075 69.96) (end 39.375 73.66) (width 0.25) (layer "F.Cu") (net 25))
 (segment (start 43.075 51.223) (end 43.075 69.96) (width 0.25) (layer "F.Cu") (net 25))
 (segment (start 41.382 49.53) (end 43.075 51.223) (width 0.25) (layer "F.Cu") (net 25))
 (segment (start 40.64 38.1) (end 39.1147 38.1) (width 0.25) (layer "F.Cu") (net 25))
 (segment (start 39.1147 38.1) (end 39.1147 48.7584) (width 0.25) (layer "F.Cu") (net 25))
 (segment (start 39.1147 48.7584) (end 39.8863 49.53) (width 0.25) (layer "F.Cu") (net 25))
 (segment (start 40.64 35.56) (end 39.1147 35.56) (width 0.25) (layer "B.Cu") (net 26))
 (segment (start 37.888 72.607) (end 36.835 73.66) (width 0.25) (layer "B.Cu") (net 26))
 (segment (start 37.3135 61.4661) (end 37.888 62.0406) (width 0.25) (layer "B.Cu") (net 26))
 (segment (start 39.1147 35.56) (end 37.3135 37.3612) (width 0.25) (layer "B.Cu") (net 26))
 (segment (start 37.3135 37.3612) (end 37.3135 61.4661) (width 0.25) (layer "B.Cu") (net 26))
 (segment (start 37.888 62.0406) (end 37.888 72.607) (width 0.25) (layer "B.Cu") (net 26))
 (segment (start 40.432 62.3683) (end 40.432 70.063) (width 0.25) (layer "B.Cu") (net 27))
 (segment (start 40.432 70.063) (end 39.375 71.12) (width 0.25) (layer "B.Cu") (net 27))
 (segment (start 42.1653 33.02) (end 42.1653 41.1435) (width 0.25) (layer "B.Cu") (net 27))
 (segment (start 42.1653 41.1435) (end 41.3988 41.91) (width 0.25) (layer "B.Cu") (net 27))
 (segment (start 40.64 33.02) (end 42.1653 33.02) (width 0.25) (layer "B.Cu") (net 27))
 (segment (start 38.2141 60.1504) (end 40.432 62.3683) (width 0.25) (layer "B.Cu") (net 27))
 (segment (start 41.3988 41.91) (end 39.8997 41.91) (width 0.25) (layer "B.Cu") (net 27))
 (segment (start 39.8997 41.91) (end 38.2141 43.5956) (width 0.25) (layer "B.Cu") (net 27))
 (segment (start 38.2141 43.5956) (end 38.2141 60.1504) (width 0.25) (layer "B.Cu") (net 27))
 (segment (start 40.64 30.48) (end 39.1147 30.48) (width 0.25) (layer "B.Cu") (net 28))
 (segment (start 35.763 70.048) (end 36.835 71.12) (width 0.25) (layer "B.Cu") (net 28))
 (segment (start 39.1147 30.48) (end 35.763 33.8317) (width 0.25) (layer "B.Cu") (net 28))
 (segment (start 35.763 33.8317) (end 35.763 70.048) (width 0.25) (layer "B.Cu") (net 28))
 (segment (start 38.6394 55.8783) (end 39.9111 57.15) (width 0.25) (layer "F.Cu") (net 29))
 (segment (start 39.1147 27.94) (end 38.6394 28.4153) (width 0.25) (layer "F.Cu") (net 29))
 (segment (start 38.6394 28.4153) (end 38.6394 55.8783) (width 0.25) (layer "F.Cu") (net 29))
 (segment (start 39.9111 57.15) (end 41.3709 57.15) (width 0.25) (layer "F.Cu") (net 29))
 (segment (start 42.1704 57.9495) (end 42.1704 65.7846) (width 0.25) (layer "F.Cu") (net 29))
 (segment (start 40.64 27.94) (end 39.1147 27.94) (width 0.25) (layer "F.Cu") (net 29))
 (segment (start 41.3709 57.15) (end 42.1704 57.9495) (width 0.25) (layer "F.Cu") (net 29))
 (segment (start 42.1704 65.7846) (end 39.375 68.58) (width 0.25) (layer "F.Cu") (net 29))
 (segment (start 36.835 27.6797) (end 36.835 66.04) (width 0.25) (layer "F.Cu") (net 30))
 (segment (start 40.64 25.4) (end 39.1147 25.4) (width 0.25) (layer "F.Cu") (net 30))
 (segment (start 39.1147 25.4) (end 36.835 27.6797) (width 0.25) (layer "F.Cu") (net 30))
 (segment (start 35.7932 26.1815) (end 35.7932 67.5382) (width 0.25) (layer "F.Cu") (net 31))
 (segment (start 40.64 22.86) (end 39.1147 22.86) (width 0.25) (layer "F.Cu") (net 31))
 (segment (start 35.7932 67.5382) (end 36.835 68.58) (width 0.25) (layer "F.Cu") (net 31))
 (segment (start 39.1147 22.86) (end 35.7932 26.1815) (width 0.25) (layer "F.Cu") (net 31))
 (segment (start 34.295 25.1397) (end 34.295 66.04) (width 0.25) (layer "F.Cu") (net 32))
 (segment (start 39.1147 20.32) (end 34.295 25.1397) (width 0.25) (layer "F.Cu") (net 32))
 (segment (start 40.64 20.32) (end 39.1147 20.32) (width 0.25) (layer "F.Cu") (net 32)))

